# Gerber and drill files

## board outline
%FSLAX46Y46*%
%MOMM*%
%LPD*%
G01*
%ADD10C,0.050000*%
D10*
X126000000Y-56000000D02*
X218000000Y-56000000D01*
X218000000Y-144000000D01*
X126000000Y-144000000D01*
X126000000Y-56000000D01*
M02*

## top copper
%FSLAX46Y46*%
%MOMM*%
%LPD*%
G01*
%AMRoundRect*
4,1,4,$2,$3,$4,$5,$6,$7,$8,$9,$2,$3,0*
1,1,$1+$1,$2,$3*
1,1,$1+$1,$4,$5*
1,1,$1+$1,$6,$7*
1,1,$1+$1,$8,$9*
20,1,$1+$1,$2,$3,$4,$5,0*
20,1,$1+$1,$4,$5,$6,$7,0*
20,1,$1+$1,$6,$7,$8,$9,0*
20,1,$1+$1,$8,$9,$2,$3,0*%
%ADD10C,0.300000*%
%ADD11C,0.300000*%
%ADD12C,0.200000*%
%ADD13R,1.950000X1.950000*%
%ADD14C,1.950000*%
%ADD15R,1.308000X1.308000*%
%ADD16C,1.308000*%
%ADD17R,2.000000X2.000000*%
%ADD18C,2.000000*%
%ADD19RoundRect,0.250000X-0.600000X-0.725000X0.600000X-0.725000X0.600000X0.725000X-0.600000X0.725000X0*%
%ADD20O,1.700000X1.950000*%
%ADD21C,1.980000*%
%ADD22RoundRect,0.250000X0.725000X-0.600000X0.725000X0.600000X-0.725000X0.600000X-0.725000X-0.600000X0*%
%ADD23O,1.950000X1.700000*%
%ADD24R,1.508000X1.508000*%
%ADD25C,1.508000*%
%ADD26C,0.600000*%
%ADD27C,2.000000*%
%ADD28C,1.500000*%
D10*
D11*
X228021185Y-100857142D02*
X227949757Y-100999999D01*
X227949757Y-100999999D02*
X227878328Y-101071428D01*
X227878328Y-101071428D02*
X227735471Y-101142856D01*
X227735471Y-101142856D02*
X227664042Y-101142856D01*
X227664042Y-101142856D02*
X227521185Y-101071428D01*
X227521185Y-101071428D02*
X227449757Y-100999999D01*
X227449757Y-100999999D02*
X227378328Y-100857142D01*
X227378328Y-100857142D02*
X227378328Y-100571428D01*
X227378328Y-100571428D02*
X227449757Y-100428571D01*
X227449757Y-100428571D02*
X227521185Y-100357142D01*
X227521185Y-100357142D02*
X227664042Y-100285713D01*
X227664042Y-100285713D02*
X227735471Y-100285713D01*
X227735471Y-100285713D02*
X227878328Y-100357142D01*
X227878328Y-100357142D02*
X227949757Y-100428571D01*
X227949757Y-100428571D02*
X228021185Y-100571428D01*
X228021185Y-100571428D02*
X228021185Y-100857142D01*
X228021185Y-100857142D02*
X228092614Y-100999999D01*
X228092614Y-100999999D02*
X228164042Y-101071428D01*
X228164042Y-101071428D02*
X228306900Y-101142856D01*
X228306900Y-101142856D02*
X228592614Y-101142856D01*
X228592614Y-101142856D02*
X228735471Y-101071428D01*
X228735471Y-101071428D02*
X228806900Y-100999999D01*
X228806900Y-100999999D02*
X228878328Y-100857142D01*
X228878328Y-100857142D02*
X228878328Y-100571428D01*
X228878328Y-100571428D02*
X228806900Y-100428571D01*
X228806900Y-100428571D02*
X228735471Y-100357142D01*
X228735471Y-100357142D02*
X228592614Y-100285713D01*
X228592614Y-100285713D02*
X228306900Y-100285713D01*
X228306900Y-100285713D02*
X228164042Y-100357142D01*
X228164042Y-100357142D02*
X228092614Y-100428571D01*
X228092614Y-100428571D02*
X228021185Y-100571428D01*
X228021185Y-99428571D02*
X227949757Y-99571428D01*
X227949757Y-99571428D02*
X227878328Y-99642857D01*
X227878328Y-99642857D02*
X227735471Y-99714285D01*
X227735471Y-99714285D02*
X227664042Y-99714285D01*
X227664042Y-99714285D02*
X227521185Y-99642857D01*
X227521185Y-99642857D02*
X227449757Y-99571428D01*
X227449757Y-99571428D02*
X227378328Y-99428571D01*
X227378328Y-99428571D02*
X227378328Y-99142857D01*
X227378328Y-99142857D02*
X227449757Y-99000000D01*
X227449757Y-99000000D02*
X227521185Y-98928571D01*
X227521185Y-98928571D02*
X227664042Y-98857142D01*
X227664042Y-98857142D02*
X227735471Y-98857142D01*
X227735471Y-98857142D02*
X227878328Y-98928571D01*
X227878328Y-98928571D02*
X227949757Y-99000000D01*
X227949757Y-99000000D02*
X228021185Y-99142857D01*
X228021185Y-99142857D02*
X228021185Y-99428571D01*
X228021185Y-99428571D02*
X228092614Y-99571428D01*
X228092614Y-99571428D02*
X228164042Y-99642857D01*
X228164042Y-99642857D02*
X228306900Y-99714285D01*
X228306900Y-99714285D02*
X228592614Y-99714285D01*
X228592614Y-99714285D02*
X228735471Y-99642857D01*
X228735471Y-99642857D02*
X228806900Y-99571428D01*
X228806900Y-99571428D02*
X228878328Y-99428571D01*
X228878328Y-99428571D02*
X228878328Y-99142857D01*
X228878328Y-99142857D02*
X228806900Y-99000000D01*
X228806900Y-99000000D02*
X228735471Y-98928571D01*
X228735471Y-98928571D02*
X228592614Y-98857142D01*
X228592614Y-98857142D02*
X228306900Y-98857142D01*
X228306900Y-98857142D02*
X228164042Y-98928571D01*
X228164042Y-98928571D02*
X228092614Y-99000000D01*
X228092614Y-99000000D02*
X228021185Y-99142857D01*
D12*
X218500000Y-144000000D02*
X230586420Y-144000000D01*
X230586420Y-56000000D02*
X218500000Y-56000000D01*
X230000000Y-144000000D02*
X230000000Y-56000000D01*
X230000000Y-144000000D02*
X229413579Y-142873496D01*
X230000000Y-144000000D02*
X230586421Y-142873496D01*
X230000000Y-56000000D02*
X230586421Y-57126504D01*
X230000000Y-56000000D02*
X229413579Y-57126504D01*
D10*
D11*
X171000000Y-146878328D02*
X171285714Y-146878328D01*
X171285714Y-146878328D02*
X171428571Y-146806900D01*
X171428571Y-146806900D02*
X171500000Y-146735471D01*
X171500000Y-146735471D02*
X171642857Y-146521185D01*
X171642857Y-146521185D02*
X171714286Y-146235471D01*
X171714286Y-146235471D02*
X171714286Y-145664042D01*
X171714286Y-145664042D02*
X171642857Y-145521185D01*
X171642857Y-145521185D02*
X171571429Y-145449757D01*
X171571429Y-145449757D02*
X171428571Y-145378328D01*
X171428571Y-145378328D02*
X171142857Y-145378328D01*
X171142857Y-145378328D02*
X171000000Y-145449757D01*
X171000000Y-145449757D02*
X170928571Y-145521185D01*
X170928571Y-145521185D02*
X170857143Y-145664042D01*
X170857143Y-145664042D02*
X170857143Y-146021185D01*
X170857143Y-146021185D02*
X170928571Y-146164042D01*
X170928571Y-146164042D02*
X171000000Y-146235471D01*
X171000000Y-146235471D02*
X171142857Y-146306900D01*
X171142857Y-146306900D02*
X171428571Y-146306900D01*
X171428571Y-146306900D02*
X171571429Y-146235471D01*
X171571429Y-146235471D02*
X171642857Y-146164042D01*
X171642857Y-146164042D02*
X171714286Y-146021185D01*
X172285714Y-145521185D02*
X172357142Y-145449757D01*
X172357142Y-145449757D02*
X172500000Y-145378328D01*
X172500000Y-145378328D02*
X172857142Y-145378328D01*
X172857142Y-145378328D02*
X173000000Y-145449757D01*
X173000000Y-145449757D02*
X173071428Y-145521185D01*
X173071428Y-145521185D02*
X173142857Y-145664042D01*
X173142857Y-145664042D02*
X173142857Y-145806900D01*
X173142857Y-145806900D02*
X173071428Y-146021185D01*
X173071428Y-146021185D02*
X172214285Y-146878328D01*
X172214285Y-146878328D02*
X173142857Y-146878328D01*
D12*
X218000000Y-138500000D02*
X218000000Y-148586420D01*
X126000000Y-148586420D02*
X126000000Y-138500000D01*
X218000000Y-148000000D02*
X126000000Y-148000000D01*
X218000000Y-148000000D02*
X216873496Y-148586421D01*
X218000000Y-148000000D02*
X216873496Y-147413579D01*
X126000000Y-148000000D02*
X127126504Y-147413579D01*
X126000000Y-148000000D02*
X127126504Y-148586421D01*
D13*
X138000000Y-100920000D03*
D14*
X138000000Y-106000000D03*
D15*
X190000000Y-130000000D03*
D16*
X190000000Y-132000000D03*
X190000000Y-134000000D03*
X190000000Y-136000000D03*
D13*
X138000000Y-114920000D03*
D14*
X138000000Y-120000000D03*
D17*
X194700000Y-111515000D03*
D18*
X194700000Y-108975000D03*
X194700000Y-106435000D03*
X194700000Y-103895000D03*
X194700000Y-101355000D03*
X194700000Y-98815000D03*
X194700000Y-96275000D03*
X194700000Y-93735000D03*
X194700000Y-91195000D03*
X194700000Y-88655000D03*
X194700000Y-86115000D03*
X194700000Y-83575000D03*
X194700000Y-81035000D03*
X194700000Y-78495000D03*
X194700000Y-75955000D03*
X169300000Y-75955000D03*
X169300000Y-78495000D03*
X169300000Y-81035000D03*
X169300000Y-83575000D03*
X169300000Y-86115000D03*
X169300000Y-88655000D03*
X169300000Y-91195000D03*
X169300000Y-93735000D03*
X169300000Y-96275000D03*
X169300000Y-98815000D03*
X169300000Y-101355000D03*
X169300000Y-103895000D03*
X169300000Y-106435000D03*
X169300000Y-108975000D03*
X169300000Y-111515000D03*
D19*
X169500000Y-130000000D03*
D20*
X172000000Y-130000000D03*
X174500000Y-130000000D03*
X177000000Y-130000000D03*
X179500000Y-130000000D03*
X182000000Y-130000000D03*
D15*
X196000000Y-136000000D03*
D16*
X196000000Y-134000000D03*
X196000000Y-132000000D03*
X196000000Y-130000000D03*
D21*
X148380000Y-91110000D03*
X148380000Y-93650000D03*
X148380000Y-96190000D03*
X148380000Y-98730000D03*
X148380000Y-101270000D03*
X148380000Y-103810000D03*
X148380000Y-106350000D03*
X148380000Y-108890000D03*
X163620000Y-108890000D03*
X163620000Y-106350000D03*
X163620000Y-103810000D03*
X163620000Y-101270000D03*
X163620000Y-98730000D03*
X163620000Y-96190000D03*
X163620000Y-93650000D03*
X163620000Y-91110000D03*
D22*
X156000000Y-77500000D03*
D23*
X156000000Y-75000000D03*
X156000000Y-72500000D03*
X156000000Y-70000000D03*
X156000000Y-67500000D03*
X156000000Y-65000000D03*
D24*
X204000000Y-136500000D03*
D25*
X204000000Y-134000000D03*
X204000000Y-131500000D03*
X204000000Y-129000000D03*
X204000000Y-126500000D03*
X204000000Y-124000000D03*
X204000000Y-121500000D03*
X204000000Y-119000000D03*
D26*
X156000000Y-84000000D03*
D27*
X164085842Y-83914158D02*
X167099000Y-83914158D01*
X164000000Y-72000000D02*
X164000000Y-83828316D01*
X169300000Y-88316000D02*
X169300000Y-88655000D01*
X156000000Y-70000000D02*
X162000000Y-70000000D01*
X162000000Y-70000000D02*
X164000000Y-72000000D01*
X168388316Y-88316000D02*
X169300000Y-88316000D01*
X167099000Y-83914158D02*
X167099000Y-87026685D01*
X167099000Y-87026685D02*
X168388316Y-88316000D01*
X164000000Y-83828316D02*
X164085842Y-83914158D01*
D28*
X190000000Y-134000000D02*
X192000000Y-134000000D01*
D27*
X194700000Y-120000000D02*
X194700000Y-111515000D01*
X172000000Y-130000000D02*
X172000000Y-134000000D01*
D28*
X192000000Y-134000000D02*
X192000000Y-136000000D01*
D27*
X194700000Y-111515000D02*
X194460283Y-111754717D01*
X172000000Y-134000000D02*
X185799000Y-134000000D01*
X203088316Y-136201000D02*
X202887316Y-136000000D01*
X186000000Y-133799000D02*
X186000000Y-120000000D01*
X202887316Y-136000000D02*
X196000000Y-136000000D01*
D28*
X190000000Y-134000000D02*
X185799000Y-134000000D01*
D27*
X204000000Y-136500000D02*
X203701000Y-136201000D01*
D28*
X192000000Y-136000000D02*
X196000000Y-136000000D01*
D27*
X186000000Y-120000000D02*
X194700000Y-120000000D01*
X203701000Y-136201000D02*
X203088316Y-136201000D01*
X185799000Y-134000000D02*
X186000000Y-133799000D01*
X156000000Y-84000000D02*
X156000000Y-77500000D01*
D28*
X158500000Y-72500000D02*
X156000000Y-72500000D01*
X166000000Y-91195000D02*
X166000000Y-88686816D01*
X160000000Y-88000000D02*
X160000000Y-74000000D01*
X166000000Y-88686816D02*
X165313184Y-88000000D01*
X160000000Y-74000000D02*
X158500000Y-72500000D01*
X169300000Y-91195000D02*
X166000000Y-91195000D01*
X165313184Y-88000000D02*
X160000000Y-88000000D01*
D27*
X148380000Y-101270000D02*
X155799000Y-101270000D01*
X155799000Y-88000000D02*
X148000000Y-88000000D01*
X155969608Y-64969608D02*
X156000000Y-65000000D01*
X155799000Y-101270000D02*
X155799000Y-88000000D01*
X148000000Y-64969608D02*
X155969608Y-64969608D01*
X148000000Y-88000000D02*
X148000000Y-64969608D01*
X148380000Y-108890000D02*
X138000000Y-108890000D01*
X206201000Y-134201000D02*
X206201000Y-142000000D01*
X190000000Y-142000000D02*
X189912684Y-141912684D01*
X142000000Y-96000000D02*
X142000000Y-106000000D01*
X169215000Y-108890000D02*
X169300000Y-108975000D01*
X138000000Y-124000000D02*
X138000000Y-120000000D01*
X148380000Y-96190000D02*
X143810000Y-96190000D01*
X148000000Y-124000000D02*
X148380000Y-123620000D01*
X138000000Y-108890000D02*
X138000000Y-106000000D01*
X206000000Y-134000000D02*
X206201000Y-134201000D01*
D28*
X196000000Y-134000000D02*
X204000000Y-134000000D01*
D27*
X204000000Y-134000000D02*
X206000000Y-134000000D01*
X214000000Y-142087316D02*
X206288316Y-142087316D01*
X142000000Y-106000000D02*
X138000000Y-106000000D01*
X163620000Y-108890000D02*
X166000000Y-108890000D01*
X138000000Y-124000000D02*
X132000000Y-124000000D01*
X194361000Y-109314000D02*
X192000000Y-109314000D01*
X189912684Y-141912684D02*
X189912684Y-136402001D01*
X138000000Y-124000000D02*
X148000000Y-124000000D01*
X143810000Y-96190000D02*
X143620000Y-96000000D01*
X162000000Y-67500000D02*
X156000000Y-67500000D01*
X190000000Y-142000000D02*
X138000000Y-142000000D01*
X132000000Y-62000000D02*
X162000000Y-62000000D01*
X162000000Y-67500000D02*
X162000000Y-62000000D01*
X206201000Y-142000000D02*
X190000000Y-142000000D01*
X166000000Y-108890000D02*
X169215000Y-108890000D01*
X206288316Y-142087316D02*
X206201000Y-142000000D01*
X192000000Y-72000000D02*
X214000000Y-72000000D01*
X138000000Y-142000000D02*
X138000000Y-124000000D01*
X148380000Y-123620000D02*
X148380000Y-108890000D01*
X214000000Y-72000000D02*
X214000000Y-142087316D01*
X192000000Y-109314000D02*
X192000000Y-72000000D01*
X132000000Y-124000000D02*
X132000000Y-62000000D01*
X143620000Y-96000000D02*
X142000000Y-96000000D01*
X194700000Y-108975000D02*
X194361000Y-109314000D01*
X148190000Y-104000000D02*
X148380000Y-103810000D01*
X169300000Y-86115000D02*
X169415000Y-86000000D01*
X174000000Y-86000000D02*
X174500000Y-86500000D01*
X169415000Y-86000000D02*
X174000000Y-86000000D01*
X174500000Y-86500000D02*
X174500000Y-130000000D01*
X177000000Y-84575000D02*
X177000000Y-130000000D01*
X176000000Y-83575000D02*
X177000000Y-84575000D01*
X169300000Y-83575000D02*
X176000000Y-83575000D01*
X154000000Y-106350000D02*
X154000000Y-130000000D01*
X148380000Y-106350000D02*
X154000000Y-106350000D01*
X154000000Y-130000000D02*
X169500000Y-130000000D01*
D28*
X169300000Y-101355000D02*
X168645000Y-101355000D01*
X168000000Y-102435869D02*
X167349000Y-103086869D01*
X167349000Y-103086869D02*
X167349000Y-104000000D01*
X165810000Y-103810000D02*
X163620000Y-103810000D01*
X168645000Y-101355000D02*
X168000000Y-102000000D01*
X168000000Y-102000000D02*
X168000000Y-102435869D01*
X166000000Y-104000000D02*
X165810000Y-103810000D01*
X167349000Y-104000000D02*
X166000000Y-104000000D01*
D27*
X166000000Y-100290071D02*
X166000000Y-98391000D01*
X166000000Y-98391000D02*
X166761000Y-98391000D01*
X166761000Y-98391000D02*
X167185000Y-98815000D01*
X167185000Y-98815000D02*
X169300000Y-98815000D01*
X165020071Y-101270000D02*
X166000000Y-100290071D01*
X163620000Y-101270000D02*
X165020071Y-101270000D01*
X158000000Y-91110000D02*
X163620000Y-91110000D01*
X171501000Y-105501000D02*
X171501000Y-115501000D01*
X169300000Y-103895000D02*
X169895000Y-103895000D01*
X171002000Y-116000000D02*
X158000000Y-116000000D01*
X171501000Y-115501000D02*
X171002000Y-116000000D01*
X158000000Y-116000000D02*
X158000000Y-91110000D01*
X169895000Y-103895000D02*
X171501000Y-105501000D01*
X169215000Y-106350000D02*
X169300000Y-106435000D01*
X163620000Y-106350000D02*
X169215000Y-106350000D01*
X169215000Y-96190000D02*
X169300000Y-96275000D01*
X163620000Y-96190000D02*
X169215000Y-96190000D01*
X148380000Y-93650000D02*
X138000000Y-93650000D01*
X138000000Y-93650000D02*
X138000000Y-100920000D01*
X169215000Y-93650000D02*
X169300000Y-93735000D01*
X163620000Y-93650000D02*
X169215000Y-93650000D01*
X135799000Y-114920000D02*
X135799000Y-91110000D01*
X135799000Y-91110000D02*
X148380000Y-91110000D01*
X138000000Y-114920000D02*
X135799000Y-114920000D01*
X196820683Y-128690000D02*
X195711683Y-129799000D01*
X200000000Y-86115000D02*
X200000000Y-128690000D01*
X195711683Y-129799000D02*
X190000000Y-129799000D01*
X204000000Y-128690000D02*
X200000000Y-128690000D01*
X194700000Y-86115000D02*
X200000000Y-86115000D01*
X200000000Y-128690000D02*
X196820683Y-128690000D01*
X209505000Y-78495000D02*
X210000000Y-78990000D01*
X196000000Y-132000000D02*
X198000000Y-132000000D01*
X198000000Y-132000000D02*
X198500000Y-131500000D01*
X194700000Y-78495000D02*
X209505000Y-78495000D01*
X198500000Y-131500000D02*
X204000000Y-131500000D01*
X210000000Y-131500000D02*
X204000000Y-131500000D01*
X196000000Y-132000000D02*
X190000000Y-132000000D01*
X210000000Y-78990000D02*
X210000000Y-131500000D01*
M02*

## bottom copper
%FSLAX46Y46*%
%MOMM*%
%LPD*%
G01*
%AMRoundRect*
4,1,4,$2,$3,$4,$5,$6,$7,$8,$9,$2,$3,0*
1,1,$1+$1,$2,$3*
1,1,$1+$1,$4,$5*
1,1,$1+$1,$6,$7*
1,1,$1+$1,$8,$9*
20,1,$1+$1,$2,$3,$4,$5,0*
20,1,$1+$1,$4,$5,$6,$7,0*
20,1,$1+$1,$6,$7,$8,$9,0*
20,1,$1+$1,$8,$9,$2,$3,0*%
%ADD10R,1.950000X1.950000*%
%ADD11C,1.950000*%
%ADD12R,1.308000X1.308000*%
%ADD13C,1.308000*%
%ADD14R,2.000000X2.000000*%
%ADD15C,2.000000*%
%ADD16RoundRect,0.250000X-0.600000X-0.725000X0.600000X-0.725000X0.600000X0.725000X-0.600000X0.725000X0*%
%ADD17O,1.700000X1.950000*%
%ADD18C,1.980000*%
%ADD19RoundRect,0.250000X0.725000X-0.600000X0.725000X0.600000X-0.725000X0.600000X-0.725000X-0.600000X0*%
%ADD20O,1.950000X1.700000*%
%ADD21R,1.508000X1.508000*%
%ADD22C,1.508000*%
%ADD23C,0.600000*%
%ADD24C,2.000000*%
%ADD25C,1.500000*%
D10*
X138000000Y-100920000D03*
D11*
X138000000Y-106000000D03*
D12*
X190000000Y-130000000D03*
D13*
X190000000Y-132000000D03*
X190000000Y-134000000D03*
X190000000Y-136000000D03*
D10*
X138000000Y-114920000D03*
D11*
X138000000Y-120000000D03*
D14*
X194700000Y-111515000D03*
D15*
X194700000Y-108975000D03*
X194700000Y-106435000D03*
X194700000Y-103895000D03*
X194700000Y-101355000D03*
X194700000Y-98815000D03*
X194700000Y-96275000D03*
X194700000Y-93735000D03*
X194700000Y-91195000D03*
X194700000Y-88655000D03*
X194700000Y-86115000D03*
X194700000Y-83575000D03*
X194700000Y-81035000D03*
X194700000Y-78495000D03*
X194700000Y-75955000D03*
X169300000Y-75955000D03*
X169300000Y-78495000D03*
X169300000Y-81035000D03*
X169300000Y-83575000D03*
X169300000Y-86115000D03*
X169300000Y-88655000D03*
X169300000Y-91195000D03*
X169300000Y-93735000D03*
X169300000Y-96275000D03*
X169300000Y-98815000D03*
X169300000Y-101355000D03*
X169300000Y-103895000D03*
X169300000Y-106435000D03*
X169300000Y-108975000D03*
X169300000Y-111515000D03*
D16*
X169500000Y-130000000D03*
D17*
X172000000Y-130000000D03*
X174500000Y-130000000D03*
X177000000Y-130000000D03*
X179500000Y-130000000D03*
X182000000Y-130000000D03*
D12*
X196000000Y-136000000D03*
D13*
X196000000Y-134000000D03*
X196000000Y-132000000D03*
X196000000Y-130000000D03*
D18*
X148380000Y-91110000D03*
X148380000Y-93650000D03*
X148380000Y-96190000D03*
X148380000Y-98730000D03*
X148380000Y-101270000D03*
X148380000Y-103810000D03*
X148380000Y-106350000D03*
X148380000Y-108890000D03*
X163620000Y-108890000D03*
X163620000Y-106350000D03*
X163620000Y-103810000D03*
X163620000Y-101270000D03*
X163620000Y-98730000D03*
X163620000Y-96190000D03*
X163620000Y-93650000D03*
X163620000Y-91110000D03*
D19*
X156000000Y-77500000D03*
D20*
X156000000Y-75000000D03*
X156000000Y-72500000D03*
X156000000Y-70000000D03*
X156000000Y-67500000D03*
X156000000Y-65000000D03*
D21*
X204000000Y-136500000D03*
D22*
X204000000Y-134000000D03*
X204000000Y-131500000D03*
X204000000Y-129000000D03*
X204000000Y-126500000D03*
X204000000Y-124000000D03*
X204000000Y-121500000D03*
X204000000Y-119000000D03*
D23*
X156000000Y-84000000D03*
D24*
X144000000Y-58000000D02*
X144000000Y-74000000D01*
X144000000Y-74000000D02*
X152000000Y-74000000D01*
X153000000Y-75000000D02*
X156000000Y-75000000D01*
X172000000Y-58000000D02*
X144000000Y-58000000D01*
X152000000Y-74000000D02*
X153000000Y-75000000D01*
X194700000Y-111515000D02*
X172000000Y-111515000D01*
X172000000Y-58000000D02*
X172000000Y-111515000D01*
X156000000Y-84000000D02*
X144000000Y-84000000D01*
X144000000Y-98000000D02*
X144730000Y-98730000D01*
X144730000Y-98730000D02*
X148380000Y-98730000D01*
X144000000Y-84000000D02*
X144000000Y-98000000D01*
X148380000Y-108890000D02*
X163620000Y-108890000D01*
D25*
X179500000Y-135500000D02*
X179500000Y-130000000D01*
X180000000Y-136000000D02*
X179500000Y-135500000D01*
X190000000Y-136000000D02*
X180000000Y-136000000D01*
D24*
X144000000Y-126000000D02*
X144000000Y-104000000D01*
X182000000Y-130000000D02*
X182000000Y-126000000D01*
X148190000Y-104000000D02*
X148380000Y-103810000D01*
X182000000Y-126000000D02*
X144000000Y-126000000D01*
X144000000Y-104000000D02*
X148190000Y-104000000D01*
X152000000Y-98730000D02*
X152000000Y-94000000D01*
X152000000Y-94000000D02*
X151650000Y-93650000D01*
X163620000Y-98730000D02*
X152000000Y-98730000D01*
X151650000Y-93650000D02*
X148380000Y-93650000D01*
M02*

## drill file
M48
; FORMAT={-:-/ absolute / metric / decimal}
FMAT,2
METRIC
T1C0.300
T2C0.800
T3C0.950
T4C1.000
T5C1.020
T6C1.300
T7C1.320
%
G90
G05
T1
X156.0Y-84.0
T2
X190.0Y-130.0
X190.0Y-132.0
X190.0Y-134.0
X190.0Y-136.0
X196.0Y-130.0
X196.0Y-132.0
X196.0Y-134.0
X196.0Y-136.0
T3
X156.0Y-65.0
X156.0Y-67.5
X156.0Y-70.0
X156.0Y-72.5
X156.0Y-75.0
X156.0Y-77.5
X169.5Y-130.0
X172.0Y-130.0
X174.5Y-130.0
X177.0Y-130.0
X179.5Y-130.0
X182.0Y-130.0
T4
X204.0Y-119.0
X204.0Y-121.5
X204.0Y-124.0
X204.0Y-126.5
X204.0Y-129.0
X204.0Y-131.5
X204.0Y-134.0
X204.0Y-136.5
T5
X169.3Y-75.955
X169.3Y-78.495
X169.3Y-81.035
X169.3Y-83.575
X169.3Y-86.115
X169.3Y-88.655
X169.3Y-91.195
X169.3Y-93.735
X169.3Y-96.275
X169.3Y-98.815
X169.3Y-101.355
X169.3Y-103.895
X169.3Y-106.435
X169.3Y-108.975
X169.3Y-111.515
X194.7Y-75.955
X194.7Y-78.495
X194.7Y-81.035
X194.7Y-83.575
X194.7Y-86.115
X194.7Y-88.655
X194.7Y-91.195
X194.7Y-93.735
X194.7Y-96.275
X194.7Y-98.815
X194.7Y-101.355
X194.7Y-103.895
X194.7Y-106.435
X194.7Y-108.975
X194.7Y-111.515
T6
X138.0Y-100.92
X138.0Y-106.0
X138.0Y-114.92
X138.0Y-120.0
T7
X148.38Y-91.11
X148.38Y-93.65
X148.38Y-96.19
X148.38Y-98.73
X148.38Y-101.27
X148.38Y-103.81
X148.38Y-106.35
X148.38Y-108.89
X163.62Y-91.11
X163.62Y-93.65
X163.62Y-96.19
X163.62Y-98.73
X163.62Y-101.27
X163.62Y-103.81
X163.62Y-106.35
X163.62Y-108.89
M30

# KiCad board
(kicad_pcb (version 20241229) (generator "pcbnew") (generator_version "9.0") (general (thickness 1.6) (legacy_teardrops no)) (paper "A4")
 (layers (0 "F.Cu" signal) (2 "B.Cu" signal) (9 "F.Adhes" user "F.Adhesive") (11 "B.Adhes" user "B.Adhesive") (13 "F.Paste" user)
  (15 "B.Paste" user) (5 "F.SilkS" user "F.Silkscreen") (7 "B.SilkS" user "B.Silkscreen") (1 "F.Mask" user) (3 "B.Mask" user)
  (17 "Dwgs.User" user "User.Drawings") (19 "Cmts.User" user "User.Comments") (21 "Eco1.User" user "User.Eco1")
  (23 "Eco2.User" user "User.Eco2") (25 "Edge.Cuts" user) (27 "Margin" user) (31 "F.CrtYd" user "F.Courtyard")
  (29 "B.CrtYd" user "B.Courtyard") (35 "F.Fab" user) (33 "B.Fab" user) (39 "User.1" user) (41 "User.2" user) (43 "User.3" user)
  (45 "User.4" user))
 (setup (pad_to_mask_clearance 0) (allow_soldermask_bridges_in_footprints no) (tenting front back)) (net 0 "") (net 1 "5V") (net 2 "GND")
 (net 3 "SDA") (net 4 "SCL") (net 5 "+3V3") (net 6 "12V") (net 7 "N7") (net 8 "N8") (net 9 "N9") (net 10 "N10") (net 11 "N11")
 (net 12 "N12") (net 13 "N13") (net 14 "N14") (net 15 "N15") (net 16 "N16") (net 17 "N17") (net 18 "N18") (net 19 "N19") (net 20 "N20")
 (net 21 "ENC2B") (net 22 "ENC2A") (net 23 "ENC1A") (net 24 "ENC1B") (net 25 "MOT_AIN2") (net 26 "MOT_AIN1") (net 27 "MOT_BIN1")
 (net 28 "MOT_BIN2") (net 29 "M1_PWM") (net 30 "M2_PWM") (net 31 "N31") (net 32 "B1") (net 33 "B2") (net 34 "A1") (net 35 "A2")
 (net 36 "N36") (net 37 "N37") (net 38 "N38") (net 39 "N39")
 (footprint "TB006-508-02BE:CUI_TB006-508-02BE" (layer "F.Cu") (at 138 100.92 -90)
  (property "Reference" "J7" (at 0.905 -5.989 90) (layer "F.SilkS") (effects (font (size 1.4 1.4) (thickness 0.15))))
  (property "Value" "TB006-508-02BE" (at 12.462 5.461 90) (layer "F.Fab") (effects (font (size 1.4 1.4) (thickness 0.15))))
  (pad "1" thru_hole rect (at 0 0 270) (size 1.95 1.95) (drill 1.3) (layers "*.Cu" "*.Mask") (remove_unused_layers no) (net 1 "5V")
   (solder_mask_margin 0.102))
  (pad "2" thru_hole circle (at 5.08 0 270) (size 1.95 1.95) (drill 1.3) (layers "*.Cu" "*.Mask") (remove_unused_layers no) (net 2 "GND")
   (solder_mask_margin 0.102)))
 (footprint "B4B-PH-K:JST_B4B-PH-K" (layer "F.Cu") (at 189.45 133 90)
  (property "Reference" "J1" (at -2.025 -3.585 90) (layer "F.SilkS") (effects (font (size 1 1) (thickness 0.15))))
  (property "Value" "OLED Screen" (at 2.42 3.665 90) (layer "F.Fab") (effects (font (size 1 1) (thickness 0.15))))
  (pad "1" thru_hole rect (at 3 0.55 90) (size 1.308 1.308) (drill 0.8) (layers "*.Cu" "*.Mask") (remove_unused_layers no) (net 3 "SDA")
   (solder_mask_margin 0.102))
  (pad "2" thru_hole circle (at 1 0.55 90) (size 1.308 1.308) (drill 0.8) (layers "*.Cu" "*.Mask") (remove_unused_layers no) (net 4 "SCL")
   (solder_mask_margin 0.102))
  (pad "3" thru_hole circle (at -1 0.55 90) (size 1.308 1.308) (drill 0.8) (layers "*.Cu" "*.Mask") (remove_unused_layers no) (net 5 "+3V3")
   (solder_mask_margin 0.102))
  (pad "4" thru_hole circle (at -3 0.55 90) (size 1.308 1.308) (drill 0.8) (layers "*.Cu" "*.Mask") (remove_unused_layers no) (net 2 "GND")
   (solder_mask_margin 0.102)))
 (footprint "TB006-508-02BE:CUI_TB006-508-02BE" (layer "F.Cu") (at 138 114.92 -90)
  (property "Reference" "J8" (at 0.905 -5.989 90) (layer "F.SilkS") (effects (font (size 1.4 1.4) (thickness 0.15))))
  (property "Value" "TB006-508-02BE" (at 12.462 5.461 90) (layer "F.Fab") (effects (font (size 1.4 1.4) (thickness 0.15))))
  (pad "1" thru_hole rect (at 0 0 270) (size 1.95 1.95) (drill 1.3) (layers "*.Cu" "*.Mask") (remove_unused_layers no) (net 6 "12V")
   (solder_mask_margin 0.102))
  (pad "2" thru_hole circle (at 5.08 0 270) (size 1.95 1.95) (drill 1.3) (layers "*.Cu" "*.Mask") (remove_unused_layers no) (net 2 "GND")
   (solder_mask_margin 0.102)))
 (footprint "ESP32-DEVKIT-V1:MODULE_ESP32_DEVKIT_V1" (layer "F.Cu") (at 182 96 180)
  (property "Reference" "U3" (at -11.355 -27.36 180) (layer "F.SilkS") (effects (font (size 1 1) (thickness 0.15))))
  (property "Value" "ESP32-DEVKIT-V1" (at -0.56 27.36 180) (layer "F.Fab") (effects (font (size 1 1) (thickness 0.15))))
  (pad "1" thru_hole rect (at -12.7 -15.515 180) (size 2 2) (drill 1.02) (layers "*.Cu" "*.Mask") (remove_unused_layers no) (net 5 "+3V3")
   (solder_mask_margin 0.102))
  (pad "2" thru_hole circle (at -12.7 -12.975 180) (size 2 2) (drill 1.02) (layers "*.Cu" "*.Mask") (remove_unused_layers no) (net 2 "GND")
   (solder_mask_margin 0.102))
  (pad "3" thru_hole circle (at -12.7 -10.435 180) (size 2 2) (drill 1.02) (layers "*.Cu" "*.Mask") (remove_unused_layers no) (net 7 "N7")
   (solder_mask_margin 0.102))
  (pad "4" thru_hole circle (at -12.7 -7.895 180) (size 2 2) (drill 1.02) (layers "*.Cu" "*.Mask") (remove_unused_layers no) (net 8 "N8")
   (solder_mask_margin 0.102))
  (pad "5" thru_hole circle (at -12.7 -5.355 180) (size 2 2) (drill 1.02) (layers "*.Cu" "*.Mask") (remove_unused_layers no) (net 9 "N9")
   (solder_mask_margin 0.102))
  (pad "6" thru_hole circle (at -12.7 -2.815 180) (size 2 2) (drill 1.02) (layers "*.Cu" "*.Mask") (remove_unused_layers no) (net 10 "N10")
   (solder_mask_margin 0.102))
  (pad "7" thru_hole circle (at -12.7 -0.275 180) (size 2 2) (drill 1.02) (layers "*.Cu" "*.Mask") (remove_unused_layers no) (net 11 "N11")
   (solder_mask_margin 0.102))
  (pad "8" thru_hole circle (at -12.7 2.265 180) (size 2 2) (drill 1.02) (layers "*.Cu" "*.Mask") (remove_unused_layers no) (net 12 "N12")
   (solder_mask_margin 0.102))
  (pad "9" thru_hole circle (at -12.7 4.805 180) (size 2 2) (drill 1.02) (layers "*.Cu" "*.Mask") (remove_unused_layers no) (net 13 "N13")
   (solder_mask_margin 0.102))
  (pad "10" thru_hole circle (at -12.7 7.345 180) (size 2 2) (drill 1.02) (layers "*.Cu" "*.Mask") (remove_unused_layers no) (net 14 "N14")
   (solder_mask_margin 0.102))
  (pad "11" thru_hole circle (at -12.7 9.885 180) (size 2 2) (drill 1.02) (layers "*.Cu" "*.Mask") (remove_unused_layers no) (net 3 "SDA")
   (solder_mask_margin 0.102))
  (pad "12" thru_hole circle (at -12.7 12.425 180) (size 2 2) (drill 1.02) (layers "*.Cu" "*.Mask") (remove_unused_layers no) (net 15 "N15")
   (solder_mask_margin 0.102))
  (pad "13" thru_hole circle (at -12.7 14.965 180) (size 2 2) (drill 1.02) (layers "*.Cu" "*.Mask") (remove_unused_layers no) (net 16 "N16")
   (solder_mask_margin 0.102))
  (pad "14" thru_hole circle (at -12.7 17.505 180) (size 2 2) (drill 1.02) (layers "*.Cu" "*.Mask") (remove_unused_layers no) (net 4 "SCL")
   (solder_mask_margin 0.102))
  (pad "15" thru_hole circle (at -12.7 20.045 180) (size 2 2) (drill 1.02) (layers "*.Cu" "*.Mask") (remove_unused_layers no) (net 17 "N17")
   (solder_mask_margin 0.102))
  (pad "16" thru_hole circle (at 12.7 20.045 180) (size 2 2) (drill 1.02) (layers "*.Cu" "*.Mask") (remove_unused_layers no) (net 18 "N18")
   (solder_mask_margin 0.102))
  (pad "17" thru_hole circle (at 12.7 17.505 180) (size 2 2) (drill 1.02) (layers "*.Cu" "*.Mask") (remove_unused_layers no) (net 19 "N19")
   (solder_mask_margin 0.102))
  (pad "18" thru_hole circle (at 12.7 14.965 180) (size 2 2) (drill 1.02) (layers "*.Cu" "*.Mask") (remove_unused_layers no) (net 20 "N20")
   (solder_mask_margin 0.102))
  (pad "19" thru_hole circle (at 12.7 12.425 180) (size 2 2) (drill 1.02) (layers "*.Cu" "*.Mask") (remove_unused_layers no)
   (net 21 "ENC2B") (solder_mask_margin 0.102))
  (pad "20" thru_hole circle (at 12.7 9.885 180) (size 2 2) (drill 1.02) (layers "*.Cu" "*.Mask") (remove_unused_layers no) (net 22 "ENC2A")
   (solder_mask_margin 0.102))
  (pad "21" thru_hole circle (at 12.7 7.345 180) (size 2 2) (drill 1.02) (layers "*.Cu" "*.Mask") (remove_unused_layers no) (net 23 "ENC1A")
   (solder_mask_margin 0.102))
  (pad "22" thru_hole circle (at 12.7 4.805 180) (size 2 2) (drill 1.02) (layers "*.Cu" "*.Mask") (remove_unused_layers no) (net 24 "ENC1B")
   (solder_mask_margin 0.102))
  (pad "23" thru_hole circle (at 12.7 2.265 180) (size 2 2) (drill 1.02) (layers "*.Cu" "*.Mask") (remove_unused_layers no)
   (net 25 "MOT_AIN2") (solder_mask_margin 0.102))
  (pad "24" thru_hole circle (at 12.7 -0.275 180) (size 2 2) (drill 1.02) (layers "*.Cu" "*.Mask") (remove_unused_layers no)
   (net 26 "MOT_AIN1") (solder_mask_margin 0.102))
  (pad "25" thru_hole circle (at 12.7 -2.815 180) (size 2 2) (drill 1.02) (layers "*.Cu" "*.Mask") (remove_unused_layers no)
   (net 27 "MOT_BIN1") (solder_mask_margin 0.102))
  (pad "26" thru_hole circle (at 12.7 -5.355 180) (size 2 2) (drill 1.02) (layers "*.Cu" "*.Mask") (remove_unused_layers no)
   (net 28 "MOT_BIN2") (solder_mask_margin 0.102))
  (pad "27" thru_hole circle (at 12.7 -7.895 180) (size 2 2) (drill 1.02) (layers "*.Cu" "*.Mask") (remove_unused_layers no)
   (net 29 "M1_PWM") (solder_mask_margin 0.102))
  (pad "28" thru_hole circle (at 12.7 -10.435 180) (size 2 2) (drill 1.02) (layers "*.Cu" "*.Mask") (remove_unused_layers no)
   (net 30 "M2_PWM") (solder_mask_margin 0.102))
  (pad "29" thru_hole circle (at 12.7 -12.975 180) (size 2 2) (drill 1.02) (layers "*.Cu" "*.Mask") (remove_unused_layers no) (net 2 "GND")
   (solder_mask_margin 0.102))
  (pad "30" thru_hole circle (at 12.7 -15.515 180) (size 2 2) (drill 1.02) (layers "*.Cu" "*.Mask") (remove_unused_layers no) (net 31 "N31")
   (solder_mask_margin 0.102))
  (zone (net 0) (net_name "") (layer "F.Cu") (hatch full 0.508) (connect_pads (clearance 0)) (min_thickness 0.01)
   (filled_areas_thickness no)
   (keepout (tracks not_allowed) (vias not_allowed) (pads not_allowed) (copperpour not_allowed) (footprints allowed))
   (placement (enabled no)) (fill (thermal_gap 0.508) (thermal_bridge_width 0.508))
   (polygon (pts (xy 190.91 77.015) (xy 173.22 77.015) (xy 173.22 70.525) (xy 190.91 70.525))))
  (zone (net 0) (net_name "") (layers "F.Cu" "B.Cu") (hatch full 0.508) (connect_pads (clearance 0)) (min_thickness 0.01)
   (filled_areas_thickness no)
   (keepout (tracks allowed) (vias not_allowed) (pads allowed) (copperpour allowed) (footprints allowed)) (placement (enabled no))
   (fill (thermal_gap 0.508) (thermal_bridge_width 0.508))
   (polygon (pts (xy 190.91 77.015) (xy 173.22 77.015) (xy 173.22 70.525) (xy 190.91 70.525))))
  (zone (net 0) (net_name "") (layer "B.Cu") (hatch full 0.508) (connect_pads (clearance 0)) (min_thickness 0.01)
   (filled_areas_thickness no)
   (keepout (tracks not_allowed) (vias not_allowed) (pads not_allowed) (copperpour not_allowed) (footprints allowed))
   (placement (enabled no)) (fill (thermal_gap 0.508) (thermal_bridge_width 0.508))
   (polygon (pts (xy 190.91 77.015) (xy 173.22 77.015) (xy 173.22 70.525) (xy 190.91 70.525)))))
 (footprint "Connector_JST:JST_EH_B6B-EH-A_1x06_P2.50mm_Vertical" (layer "F.Cu") (at 169.5 130)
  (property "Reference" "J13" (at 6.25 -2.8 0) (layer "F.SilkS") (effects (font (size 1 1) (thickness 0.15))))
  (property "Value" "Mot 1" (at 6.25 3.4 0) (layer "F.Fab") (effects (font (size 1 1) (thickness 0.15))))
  (pad "1" thru_hole roundrect (at 0 0) (size 1.7 1.95) (drill 0.95) (layers "*.Cu" "*.Mask") (remove_unused_layers no)
   (roundrect_rratio 0.147059) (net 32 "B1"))
  (pad "2" thru_hole oval (at 2.5 0) (size 1.7 1.95) (drill 0.95) (layers "*.Cu" "*.Mask") (remove_unused_layers no) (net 5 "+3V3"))
  (pad "3" thru_hole oval (at 5 0) (size 1.7 1.95) (drill 0.95) (layers "*.Cu" "*.Mask") (remove_unused_layers no) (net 22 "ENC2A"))
  (pad "4" thru_hole oval (at 7.5 0) (size 1.7 1.95) (drill 0.95) (layers "*.Cu" "*.Mask") (remove_unused_layers no) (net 21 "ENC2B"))
  (pad "5" thru_hole oval (at 10 0) (size 1.7 1.95) (drill 0.95) (layers "*.Cu" "*.Mask") (remove_unused_layers no) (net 2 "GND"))
  (pad "6" thru_hole oval (at 12.5 0) (size 1.7 1.95) (drill 0.95) (layers "*.Cu" "*.Mask") (remove_unused_layers no) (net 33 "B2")))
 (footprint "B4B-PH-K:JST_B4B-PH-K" (layer "F.Cu") (at 196.55 133 -90)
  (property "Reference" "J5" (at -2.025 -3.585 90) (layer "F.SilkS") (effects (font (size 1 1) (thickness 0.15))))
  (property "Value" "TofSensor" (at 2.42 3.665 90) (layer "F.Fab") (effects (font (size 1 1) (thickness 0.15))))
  (pad "1" thru_hole rect (at 3 0.55 270) (size 1.308 1.308) (drill 0.8) (layers "*.Cu" "*.Mask") (remove_unused_layers no) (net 5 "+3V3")
   (solder_mask_margin 0.102))
  (pad "2" thru_hole circle (at 1 0.55 270) (size 1.308 1.308) (drill 0.8) (layers "*.Cu" "*.Mask") (remove_unused_layers no) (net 2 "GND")
   (solder_mask_margin 0.102))
  (pad "3" thru_hole circle (at -1 0.55 270) (size 1.308 1.308) (drill 0.8) (layers "*.Cu" "*.Mask") (remove_unused_layers no) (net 4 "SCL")
   (solder_mask_margin 0.102))
  (pad "4" thru_hole circle (at -3 0.55 270) (size 1.308 1.308) (drill 0.8) (layers "*.Cu" "*.Mask") (remove_unused_layers no) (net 3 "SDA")
   (solder_mask_margin 0.102)))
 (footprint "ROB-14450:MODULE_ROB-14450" (layer "F.Cu") (at 156 100)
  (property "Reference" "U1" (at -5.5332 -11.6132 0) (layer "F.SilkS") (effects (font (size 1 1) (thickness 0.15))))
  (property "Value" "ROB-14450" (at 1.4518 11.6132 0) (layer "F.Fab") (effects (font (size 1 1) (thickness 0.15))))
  (pad "1" thru_hole circle (at -7.62 -8.89) (size 1.98 1.98) (drill 1.32) (layers "*.Cu" "*.Mask") (remove_unused_layers no) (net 6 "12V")
   (solder_mask_margin 0.102))
  (pad "2" thru_hole circle (at -7.62 -6.35) (size 1.98 1.98) (drill 1.32) (layers "*.Cu" "*.Mask") (remove_unused_layers no) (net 1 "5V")
   (solder_mask_margin 0.102))
  (pad "3" thru_hole circle (at -7.62 -3.81) (size 1.98 1.98) (drill 1.32) (layers "*.Cu" "*.Mask") (remove_unused_layers no) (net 2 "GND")
   (solder_mask_margin 0.102))
  (pad "4" thru_hole circle (at -7.62 -1.27) (size 1.98 1.98) (drill 1.32) (layers "*.Cu" "*.Mask") (remove_unused_layers no) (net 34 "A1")
   (solder_mask_margin 0.102))
  (pad "5" thru_hole circle (at -7.62 1.27) (size 1.98 1.98) (drill 1.32) (layers "*.Cu" "*.Mask") (remove_unused_layers no) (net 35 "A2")
   (solder_mask_margin 0.102))
  (pad "6" thru_hole circle (at -7.62 3.81) (size 1.98 1.98) (drill 1.32) (layers "*.Cu" "*.Mask") (remove_unused_layers no) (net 33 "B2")
   (solder_mask_margin 0.102))
  (pad "7" thru_hole circle (at -7.62 6.35) (size 1.98 1.98) (drill 1.32) (layers "*.Cu" "*.Mask") (remove_unused_layers no) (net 32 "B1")
   (solder_mask_margin 0.102))
  (pad "8" thru_hole circle (at -7.62 8.89) (size 1.98 1.98) (drill 1.32) (layers "*.Cu" "*.Mask") (remove_unused_layers no) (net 2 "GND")
   (solder_mask_margin 0.102))
  (pad "9" thru_hole circle (at 7.62 8.89) (size 1.98 1.98) (drill 1.32) (layers "*.Cu" "*.Mask") (remove_unused_layers no) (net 2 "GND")
   (solder_mask_margin 0.102))
  (pad "10" thru_hole circle (at 7.62 6.35) (size 1.98 1.98) (drill 1.32) (layers "*.Cu" "*.Mask") (remove_unused_layers no)
   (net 30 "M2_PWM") (solder_mask_margin 0.102))
  (pad "11" thru_hole circle (at 7.62 3.81) (size 1.98 1.98) (drill 1.32) (layers "*.Cu" "*.Mask") (remove_unused_layers no)
   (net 28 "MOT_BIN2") (solder_mask_margin 0.102))
  (pad "12" thru_hole circle (at 7.62 1.27) (size 1.98 1.98) (drill 1.32) (layers "*.Cu" "*.Mask") (remove_unused_layers no)
   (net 27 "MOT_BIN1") (solder_mask_margin 0.102))
  (pad "13" thru_hole circle (at 7.62 -1.27) (size 1.98 1.98) (drill 1.32) (layers "*.Cu" "*.Mask") (remove_unused_layers no) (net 1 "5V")
   (solder_mask_margin 0.102))
  (pad "14" thru_hole circle (at 7.62 -3.81) (size 1.98 1.98) (drill 1.32) (layers "*.Cu" "*.Mask") (remove_unused_layers no)
   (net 26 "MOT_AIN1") (solder_mask_margin 0.102))
  (pad "15" thru_hole circle (at 7.62 -6.35) (size 1.98 1.98) (drill 1.32) (layers "*.Cu" "*.Mask") (remove_unused_layers no)
   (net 25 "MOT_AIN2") (solder_mask_margin 0.102))
  (pad "16" thru_hole circle (at 7.62 -8.89) (size 1.98 1.98) (drill 1.32) (layers "*.Cu" "*.Mask") (remove_unused_layers no)
   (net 29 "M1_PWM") (solder_mask_margin 0.102)))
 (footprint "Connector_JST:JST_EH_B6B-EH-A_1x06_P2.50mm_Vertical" (layer "F.Cu") (at 156 77.5 90)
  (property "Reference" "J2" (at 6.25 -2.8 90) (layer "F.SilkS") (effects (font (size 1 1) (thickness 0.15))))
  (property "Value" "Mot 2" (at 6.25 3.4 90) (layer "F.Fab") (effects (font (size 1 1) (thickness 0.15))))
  (pad "1" thru_hole roundrect (at 0 0 90) (size 1.7 1.95) (drill 0.95) (layers "*.Cu" "*.Mask") (remove_unused_layers no)
   (roundrect_rratio 0.147059) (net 34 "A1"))
  (pad "2" thru_hole oval (at 2.5 0 90) (size 1.7 1.95) (drill 0.95) (layers "*.Cu" "*.Mask") (remove_unused_layers no) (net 5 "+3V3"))
  (pad "3" thru_hole oval (at 5 0 90) (size 1.7 1.95) (drill 0.95) (layers "*.Cu" "*.Mask") (remove_unused_layers no) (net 24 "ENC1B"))
  (pad "4" thru_hole oval (at 7.5 0 90) (size 1.7 1.95) (drill 0.95) (layers "*.Cu" "*.Mask") (remove_unused_layers no) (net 23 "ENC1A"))
  (pad "5" thru_hole oval (at 10 0 90) (size 1.7 1.95) (drill 0.95) (layers "*.Cu" "*.Mask") (remove_unused_layers no) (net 2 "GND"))
  (pad "6" thru_hole oval (at 12.5 0 90) (size 1.7 1.95) (drill 0.95) (layers "*.Cu" "*.Mask") (remove_unused_layers no) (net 35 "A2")))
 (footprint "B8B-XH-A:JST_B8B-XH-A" (layer "F.Cu") (at 204.525 127.75 -90)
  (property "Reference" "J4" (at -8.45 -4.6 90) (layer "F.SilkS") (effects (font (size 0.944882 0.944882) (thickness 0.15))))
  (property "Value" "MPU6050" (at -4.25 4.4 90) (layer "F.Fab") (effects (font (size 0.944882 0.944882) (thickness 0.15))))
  (pad "1" thru_hole rect (at 8.75 0.525 270) (size 1.508 1.508) (drill 1) (layers "*.Cu" "*.Mask") (remove_unused_layers no) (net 5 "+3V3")
   (solder_mask_margin 0.102))
  (pad "2" thru_hole circle (at 6.25 0.525 270) (size 1.508 1.508) (drill 1) (layers "*.Cu" "*.Mask") (remove_unused_layers no)
   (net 2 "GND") (solder_mask_margin 0.102))
  (pad "3" thru_hole circle (at 3.75 0.525 270) (size 1.508 1.508) (drill 1) (layers "*.Cu" "*.Mask") (remove_unused_layers no)
   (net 4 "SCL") (solder_mask_margin 0.102))
  (pad "4" thru_hole circle (at 1.25 0.525 270) (size 1.508 1.508) (drill 1) (layers "*.Cu" "*.Mask") (remove_unused_layers no)
   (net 3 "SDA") (solder_mask_margin 0.102))
  (pad "5" thru_hole circle (at -1.25 0.525 270) (size 1.508 1.508) (drill 1) (layers "*.Cu" "*.Mask") (remove_unused_layers no)
   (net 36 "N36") (solder_mask_margin 0.102))
  (pad "6" thru_hole circle (at -3.75 0.525 270) (size 1.508 1.508) (drill 1) (layers "*.Cu" "*.Mask") (remove_unused_layers no)
   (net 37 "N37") (solder_mask_margin 0.102))
  (pad "7" thru_hole circle (at -6.25 0.525 270) (size 1.508 1.508) (drill 1) (layers "*.Cu" "*.Mask") (remove_unused_layers no)
   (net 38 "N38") (solder_mask_margin 0.102))
  (pad "8" thru_hole circle (at -8.75 0.525 270) (size 1.508 1.508) (drill 1) (layers "*.Cu" "*.Mask") (remove_unused_layers no)
   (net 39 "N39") (solder_mask_margin 0.102)))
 (gr_rect (start 126 56) (end 218 144) (stroke (width 0.05) (type default)) (fill no) (layer "Edge.Cuts"))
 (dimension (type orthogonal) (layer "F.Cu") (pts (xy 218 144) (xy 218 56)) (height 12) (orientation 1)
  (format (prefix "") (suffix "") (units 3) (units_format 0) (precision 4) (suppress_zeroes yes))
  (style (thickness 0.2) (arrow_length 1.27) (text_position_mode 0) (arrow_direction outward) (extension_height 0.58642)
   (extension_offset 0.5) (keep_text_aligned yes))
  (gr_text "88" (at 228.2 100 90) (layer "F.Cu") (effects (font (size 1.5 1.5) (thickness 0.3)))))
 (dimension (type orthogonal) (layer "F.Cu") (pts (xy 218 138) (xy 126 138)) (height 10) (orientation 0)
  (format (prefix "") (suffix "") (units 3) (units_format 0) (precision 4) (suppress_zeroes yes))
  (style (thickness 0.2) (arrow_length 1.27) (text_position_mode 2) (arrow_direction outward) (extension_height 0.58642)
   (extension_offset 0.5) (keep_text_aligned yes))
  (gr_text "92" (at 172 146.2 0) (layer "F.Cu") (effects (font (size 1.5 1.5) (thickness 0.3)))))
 (segment (start 164.085842 83.914158) (end 167.099 83.914158) (width 2) (layer "F.Cu") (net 23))
 (segment (start 164 72) (end 164 83.828316) (width 2) (layer "F.Cu") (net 23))
 (segment (start 169.3 88.316) (end 169.3 88.655) (width 2) (layer "F.Cu") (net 23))
 (segment (start 156 70) (end 162 70) (width 2) (layer "F.Cu") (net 23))
 (segment (start 162 70) (end 164 72) (width 2) (layer "F.Cu") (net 23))
 (segment (start 168.388316 88.316) (end 169.3 88.316) (width 2) (layer "F.Cu") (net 23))
 (segment (start 167.099 83.914158) (end 167.099 87.026685) (width 2) (layer "F.Cu") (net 23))
 (segment (start 167.099 87.026685) (end 168.388316 88.316) (width 2) (layer "F.Cu") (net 23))
 (segment (start 164 83.828316) (end 164.085842 83.914158) (width 2) (layer "F.Cu") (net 23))
 (segment (start 190 134) (end 192 134) (width 1.5) (layer "F.Cu") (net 5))
 (segment (start 194.7 120) (end 194.7 111.515) (width 2) (layer "F.Cu") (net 5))
 (segment (start 172 130) (end 172 134) (width 2) (layer "F.Cu") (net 5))
 (segment (start 192 134) (end 192 136) (width 1.5) (layer "F.Cu") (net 5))
 (segment (start 194.7 111.515) (end 194.460283 111.754717) (width 2) (layer "F.Cu") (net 5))
 (segment (start 172 134) (end 185.799 134) (width 2) (layer "F.Cu") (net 5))
 (segment (start 203.088316 136.201) (end 202.887316 136) (width 2) (layer "F.Cu") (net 5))
 (segment (start 186 133.799) (end 186 120) (width 2) (layer "F.Cu") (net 5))
 (segment (start 202.887316 136) (end 196 136) (width 2) (layer "F.Cu") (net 5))
 (segment (start 190 134) (end 185.799 134) (width 1.5) (layer "F.Cu") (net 5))
 (segment (start 204 136.5) (end 203.701 136.201) (width 2) (layer "F.Cu") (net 5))
 (segment (start 192 136) (end 196 136) (width 1.5) (layer "F.Cu") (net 5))
 (segment (start 186 120) (end 194.7 120) (width 2) (layer "F.Cu") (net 5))
 (segment (start 203.701 136.201) (end 203.088316 136.201) (width 2) (layer "F.Cu") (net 5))
 (segment (start 185.799 134) (end 186 133.799) (width 2) (layer "F.Cu") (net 5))
 (segment (start 144 58) (end 144 74) (width 2) (layer "B.Cu") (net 5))
 (segment (start 144 74) (end 152 74) (width 2) (layer "B.Cu") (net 5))
 (segment (start 153 75) (end 156 75) (width 2) (layer "B.Cu") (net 5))
 (segment (start 172 58) (end 144 58) (width 2) (layer "B.Cu") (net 5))
 (segment (start 152 74) (end 153 75) (width 2) (layer "B.Cu") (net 5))
 (segment (start 194.7 111.515) (end 172 111.515) (width 2) (layer "B.Cu") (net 5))
 (segment (start 172 58) (end 172 111.515) (width 2) (layer "B.Cu") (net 5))
 (segment (start 156 84) (end 156 77.5) (width 2) (layer "F.Cu") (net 34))
 (via (at 156 84) (size 0.6) (drill 0.3) (layers "F.Cu" "B.Cu") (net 34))
 (segment (start 156 84) (end 144 84) (width 2) (layer "B.Cu") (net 34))
 (segment (start 144 98) (end 144.73 98.73) (width 2) (layer "B.Cu") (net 34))
 (segment (start 144.73 98.73) (end 148.38 98.73) (width 2) (layer "B.Cu") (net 34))
 (segment (start 144 84) (end 144 98) (width 2) (layer "B.Cu") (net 34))
 (segment (start 158.5 72.5) (end 156 72.5) (width 1.5) (layer "F.Cu") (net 24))
 (segment (start 166 91.195) (end 166 88.686816) (width 1.5) (layer "F.Cu") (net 24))
 (segment (start 160 88) (end 160 74) (width 1.5) (layer "F.Cu") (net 24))
 (segment (start 166 88.686816) (end 165.313184 88) (width 1.5) (layer "F.Cu") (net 24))
 (segment (start 160 74) (end 158.5 72.5) (width 1.5) (layer "F.Cu") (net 24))
 (segment (start 169.3 91.195) (end 166 91.195) (width 1.5) (layer "F.Cu") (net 24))
 (segment (start 165.313184 88) (end 160 88) (width 1.5) (layer "F.Cu") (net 24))
 (segment (start 148.38 101.27) (end 155.799 101.27) (width 2) (layer "F.Cu") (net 35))
 (segment (start 155.799 88) (end 148 88) (width 2) (layer "F.Cu") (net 35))
 (segment (start 155.969608 64.969608) (end 156 65) (width 2) (layer "F.Cu") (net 35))
 (segment (start 155.799 101.27) (end 155.799 88) (width 2) (layer "F.Cu") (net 35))
 (segment (start 148 64.969608) (end 155.969608 64.969608) (width 2) (layer "F.Cu") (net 35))
 (segment (start 148 88) (end 148 64.969608) (width 2) (layer "F.Cu") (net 35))
 (segment (start 148.38 108.89) (end 138 108.89) (width 2) (layer "F.Cu") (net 2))
 (segment (start 206.201 134.201) (end 206.201 142) (width 2) (layer "F.Cu") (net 2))
 (segment (start 190 142) (end 189.912684 141.912684) (width 2) (layer "F.Cu") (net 2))
 (segment (start 142 96) (end 142 106) (width 2) (layer "F.Cu") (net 2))
 (segment (start 169.215 108.89) (end 169.3 108.975) (width 2) (layer "F.Cu") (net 2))
 (segment (start 138 124) (end 138 120) (width 2) (layer "F.Cu") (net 2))
 (segment (start 148.38 96.19) (end 143.81 96.19) (width 2) (layer "F.Cu") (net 2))
 (segment (start 148 124) (end 148.38 123.62) (width 2) (layer "F.Cu") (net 2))
 (segment (start 138 108.89) (end 138 106) (width 2) (layer "F.Cu") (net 2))
 (segment (start 206 134) (end 206.201 134.201) (width 2) (layer "F.Cu") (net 2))
 (segment (start 196 134) (end 204 134) (width 1.5) (layer "F.Cu") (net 2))
 (segment (start 204 134) (end 206 134) (width 2) (layer "F.Cu") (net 2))
 (segment (start 214 142.087316) (end 206.288316 142.087316) (width 2) (layer "F.Cu") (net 2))
 (segment (start 142 106) (end 138 106) (width 2) (layer "F.Cu") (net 2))
 (segment (start 163.62 108.89) (end 166 108.89) (width 2) (layer "F.Cu") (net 2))
 (segment (start 138 124) (end 132 124) (width 2) (layer "F.Cu") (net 2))
 (segment (start 194.361 109.314) (end 192 109.314) (width 2) (layer "F.Cu") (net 2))
 (segment (start 189.912684 141.912684) (end 189.912684 136.402001) (width 2) (layer "F.Cu") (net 2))
 (segment (start 138 124) (end 148 124) (width 2) (layer "F.Cu") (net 2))
 (segment (start 143.81 96.19) (end 143.62 96) (width 2) (layer "F.Cu") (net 2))
 (segment (start 162 67.5) (end 156 67.5) (width 2) (layer "F.Cu") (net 2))
 (segment (start 190 142) (end 138 142) (width 2) (layer "F.Cu") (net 2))
 (segment (start 132 62) (end 162 62) (width 2) (layer "F.Cu") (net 2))
 (segment (start 162 67.5) (end 162 62) (width 2) (layer "F.Cu") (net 2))
 (segment (start 206.201 142) (end 190 142) (width 2) (layer "F.Cu") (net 2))
 (segment (start 166 108.89) (end 169.215 108.89) (width 2) (layer "F.Cu") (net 2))
 (segment (start 206.288316 142.087316) (end 206.201 142) (width 2) (layer "F.Cu") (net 2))
 (segment (start 192 72) (end 214 72) (width 2) (layer "F.Cu") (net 2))
 (segment (start 138 142) (end 138 124) (width 2) (layer "F.Cu") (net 2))
 (segment (start 148.38 123.62) (end 148.38 108.89) (width 2) (layer "F.Cu") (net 2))
 (segment (start 214 72) (end 214 142.087316) (width 2) (layer "F.Cu") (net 2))
 (segment (start 192 109.314) (end 192 72) (width 2) (layer "F.Cu") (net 2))
 (segment (start 132 124) (end 132 62) (width 2) (layer "F.Cu") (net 2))
 (segment (start 143.62 96) (end 142 96) (width 2) (layer "F.Cu") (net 2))
 (segment (start 194.7 108.975) (end 194.361 109.314) (width 2) (layer "F.Cu") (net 2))
 (segment (start 148.38 108.89) (end 163.62 108.89) (width 2) (layer "B.Cu") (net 2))
 (segment (start 179.5 135.5) (end 179.5 130) (width 1.5) (layer "B.Cu") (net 2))
 (segment (start 180 136) (end 179.5 135.5) (width 1.5) (layer "B.Cu") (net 2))
 (segment (start 190 136) (end 180 136) (width 1.5) (layer "B.Cu") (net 2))
 (segment (start 148.19 104) (end 148.38 103.81) (width 2) (layer "F.Cu") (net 33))
 (segment (start 144 126) (end 144 104) (width 2) (layer "B.Cu") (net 33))
 (segment (start 182 130) (end 182 126) (width 2) (layer "B.Cu") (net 33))
 (segment (start 148.19 104) (end 148.38 103.81) (width 2) (layer "B.Cu") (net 33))
 (segment (start 182 126) (end 144 126) (width 2) (layer "B.Cu") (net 33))
 (segment (start 144 104) (end 148.19 104) (width 2) (layer "B.Cu") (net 33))
 (segment (start 169.3 86.115) (end 169.415 86) (width 2) (layer "F.Cu") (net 22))
 (segment (start 174 86) (end 174.5 86.5) (width 2) (layer "F.Cu") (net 22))
 (segment (start 169.415 86) (end 174 86) (width 2) (layer "F.Cu") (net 22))
 (segment (start 174.5 86.5) (end 174.5 130) (width 2) (layer "F.Cu") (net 22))
 (segment (start 177 84.575) (end 177 130) (width 2) (layer "F.Cu") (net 21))
 (segment (start 176 83.575) (end 177 84.575) (width 2) (layer "F.Cu") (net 21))
 (segment (start 169.3 83.575) (end 176 83.575) (width 2) (layer "F.Cu") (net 21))
 (segment (start 154 106.35) (end 154 130) (width 2) (layer "F.Cu") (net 32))
 (segment (start 148.38 106.35) (end 154 106.35) (width 2) (layer "F.Cu") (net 32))
 (segment (start 154 130) (end 169.5 130) (width 2) (layer "F.Cu") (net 32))
 (segment (start 169.3 101.355) (end 168.645 101.355) (width 1.5) (layer "F.Cu") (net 28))
 (segment (start 168 102.435869) (end 167.349 103.086869) (width 1.5) (layer "F.Cu") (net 28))
 (segment (start 167.349 103.086869) (end 167.349 104) (width 1.5) (layer "F.Cu") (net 28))
 (segment (start 165.81 103.81) (end 163.62 103.81) (width 1.5) (layer "F.Cu") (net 28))
 (segment (start 168.645 101.355) (end 168 102) (width 1.5) (layer "F.Cu") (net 28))
 (segment (start 168 102) (end 168 102.435869) (width 1.5) (layer "F.Cu") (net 28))
 (segment (start 166 104) (end 165.81 103.81) (width 1.5) (layer "F.Cu") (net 28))
 (segment (start 167.349 104) (end 166 104) (width 1.5) (layer "F.Cu") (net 28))
 (segment (start 166 100.290071) (end 166 98.391) (width 2) (layer "F.Cu") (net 27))
 (segment (start 166 98.391) (end 166.761 98.391) (width 2) (layer "F.Cu") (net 27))
 (segment (start 166.761 98.391) (end 167.185 98.815) (width 2) (layer "F.Cu") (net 27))
 (segment (start 167.185 98.815) (end 169.3 98.815) (width 2) (layer "F.Cu") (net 27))
 (segment (start 165.020071 101.27) (end 166 100.290071) (width 2) (layer "F.Cu") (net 27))
 (segment (start 163.62 101.27) (end 165.020071 101.27) (width 2) (layer "F.Cu") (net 27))
 (segment (start 158 91.11) (end 163.62 91.11) (width 2) (layer "F.Cu") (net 29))
 (segment (start 171.501 105.501) (end 171.501 115.501) (width 2) (layer "F.Cu") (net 29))
 (segment (start 169.3 103.895) (end 169.895 103.895) (width 2) (layer "F.Cu") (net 29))
 (segment (start 171.002 116) (end 158 116) (width 2) (layer "F.Cu") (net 29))
 (segment (start 171.501 115.501) (end 171.002 116) (width 2) (layer "F.Cu") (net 29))
 (segment (start 158 116) (end 158 91.11) (width 2) (layer "F.Cu") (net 29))
 (segment (start 169.895 103.895) (end 171.501 105.501) (width 2) (layer "F.Cu") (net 29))
 (segment (start 169.215 106.35) (end 169.3 106.435) (width 2) (layer "F.Cu") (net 30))
 (segment (start 163.62 106.35) (end 169.215 106.35) (width 2) (layer "F.Cu") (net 30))
 (segment (start 169.215 96.19) (end 169.3 96.275) (width 2) (layer "F.Cu") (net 26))
 (segment (start 163.62 96.19) (end 169.215 96.19) (width 2) (layer "F.Cu") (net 26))
 (segment (start 148.38 93.65) (end 138 93.65) (width 2) (layer "F.Cu") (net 1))
 (segment (start 138 93.65) (end 138 100.92) (width 2) (layer "F.Cu") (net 1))
 (segment (start 152 98.73) (end 152 94) (width 2) (layer "B.Cu") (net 1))
 (segment (start 152 94) (end 151.65 93.65) (width 2) (layer "B.Cu") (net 1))
 (segment (start 163.62 98.73) (end 152 98.73) (width 2) (layer "B.Cu") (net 1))
 (segment (start 151.65 93.65) (end 148.38 93.65) (width 2) (layer "B.Cu") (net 1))
 (segment (start 169.215 93.65) (end 169.3 93.735) (width 2) (layer "F.Cu") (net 25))
 (segment (start 163.62 93.65) (end 169.215 93.65) (width 2) (layer "F.Cu") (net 25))
 (segment (start 135.799 114.92) (end 135.799 91.11) (width 2) (layer "F.Cu") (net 6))
 (segment (start 135.799 91.11) (end 148.38 91.11) (width 2) (layer "F.Cu") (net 6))
 (segment (start 138 114.92) (end 135.799 114.92) (width 2) (layer "F.Cu") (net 6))
 (segment (start 196.820683 128.69) (end 195.711683 129.799) (width 2) (layer "F.Cu") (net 3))
 (segment (start 200 86.115) (end 200 128.69) (width 2) (layer "F.Cu") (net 3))
 (segment (start 195.711683 129.799) (end 190 129.799) (width 2) (layer "F.Cu") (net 3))
 (segment (start 204 128.69) (end 200 128.69) (width 2) (layer "F.Cu") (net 3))
 (segment (start 194.7 86.115) (end 200 86.115) (width 2) (layer "F.Cu") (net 3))
 (segment (start 200 128.69) (end 196.820683 128.69) (width 2) (layer "F.Cu") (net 3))
 (segment (start 209.505 78.495) (end 210 78.99) (width 2) (layer "F.Cu") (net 4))
 (segment (start 196 132) (end 198 132) (width 2) (layer "F.Cu") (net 4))
 (segment (start 198 132) (end 198.5 131.5) (width 2) (layer "F.Cu") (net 4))
 (segment (start 194.7 78.495) (end 209.505 78.495) (width 2) (layer "F.Cu") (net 4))
 (segment (start 198.5 131.5) (end 204 131.5) (width 2) (layer "F.Cu") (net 4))
 (segment (start 210 131.5) (end 204 131.5) (width 2) (layer "F.Cu") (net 4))
 (segment (start 196 132) (end 190 132) (width 2) (layer "F.Cu") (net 4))
 (segment (start 210 78.99) (end 210 131.5) (width 2) (layer "F.Cu") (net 4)))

